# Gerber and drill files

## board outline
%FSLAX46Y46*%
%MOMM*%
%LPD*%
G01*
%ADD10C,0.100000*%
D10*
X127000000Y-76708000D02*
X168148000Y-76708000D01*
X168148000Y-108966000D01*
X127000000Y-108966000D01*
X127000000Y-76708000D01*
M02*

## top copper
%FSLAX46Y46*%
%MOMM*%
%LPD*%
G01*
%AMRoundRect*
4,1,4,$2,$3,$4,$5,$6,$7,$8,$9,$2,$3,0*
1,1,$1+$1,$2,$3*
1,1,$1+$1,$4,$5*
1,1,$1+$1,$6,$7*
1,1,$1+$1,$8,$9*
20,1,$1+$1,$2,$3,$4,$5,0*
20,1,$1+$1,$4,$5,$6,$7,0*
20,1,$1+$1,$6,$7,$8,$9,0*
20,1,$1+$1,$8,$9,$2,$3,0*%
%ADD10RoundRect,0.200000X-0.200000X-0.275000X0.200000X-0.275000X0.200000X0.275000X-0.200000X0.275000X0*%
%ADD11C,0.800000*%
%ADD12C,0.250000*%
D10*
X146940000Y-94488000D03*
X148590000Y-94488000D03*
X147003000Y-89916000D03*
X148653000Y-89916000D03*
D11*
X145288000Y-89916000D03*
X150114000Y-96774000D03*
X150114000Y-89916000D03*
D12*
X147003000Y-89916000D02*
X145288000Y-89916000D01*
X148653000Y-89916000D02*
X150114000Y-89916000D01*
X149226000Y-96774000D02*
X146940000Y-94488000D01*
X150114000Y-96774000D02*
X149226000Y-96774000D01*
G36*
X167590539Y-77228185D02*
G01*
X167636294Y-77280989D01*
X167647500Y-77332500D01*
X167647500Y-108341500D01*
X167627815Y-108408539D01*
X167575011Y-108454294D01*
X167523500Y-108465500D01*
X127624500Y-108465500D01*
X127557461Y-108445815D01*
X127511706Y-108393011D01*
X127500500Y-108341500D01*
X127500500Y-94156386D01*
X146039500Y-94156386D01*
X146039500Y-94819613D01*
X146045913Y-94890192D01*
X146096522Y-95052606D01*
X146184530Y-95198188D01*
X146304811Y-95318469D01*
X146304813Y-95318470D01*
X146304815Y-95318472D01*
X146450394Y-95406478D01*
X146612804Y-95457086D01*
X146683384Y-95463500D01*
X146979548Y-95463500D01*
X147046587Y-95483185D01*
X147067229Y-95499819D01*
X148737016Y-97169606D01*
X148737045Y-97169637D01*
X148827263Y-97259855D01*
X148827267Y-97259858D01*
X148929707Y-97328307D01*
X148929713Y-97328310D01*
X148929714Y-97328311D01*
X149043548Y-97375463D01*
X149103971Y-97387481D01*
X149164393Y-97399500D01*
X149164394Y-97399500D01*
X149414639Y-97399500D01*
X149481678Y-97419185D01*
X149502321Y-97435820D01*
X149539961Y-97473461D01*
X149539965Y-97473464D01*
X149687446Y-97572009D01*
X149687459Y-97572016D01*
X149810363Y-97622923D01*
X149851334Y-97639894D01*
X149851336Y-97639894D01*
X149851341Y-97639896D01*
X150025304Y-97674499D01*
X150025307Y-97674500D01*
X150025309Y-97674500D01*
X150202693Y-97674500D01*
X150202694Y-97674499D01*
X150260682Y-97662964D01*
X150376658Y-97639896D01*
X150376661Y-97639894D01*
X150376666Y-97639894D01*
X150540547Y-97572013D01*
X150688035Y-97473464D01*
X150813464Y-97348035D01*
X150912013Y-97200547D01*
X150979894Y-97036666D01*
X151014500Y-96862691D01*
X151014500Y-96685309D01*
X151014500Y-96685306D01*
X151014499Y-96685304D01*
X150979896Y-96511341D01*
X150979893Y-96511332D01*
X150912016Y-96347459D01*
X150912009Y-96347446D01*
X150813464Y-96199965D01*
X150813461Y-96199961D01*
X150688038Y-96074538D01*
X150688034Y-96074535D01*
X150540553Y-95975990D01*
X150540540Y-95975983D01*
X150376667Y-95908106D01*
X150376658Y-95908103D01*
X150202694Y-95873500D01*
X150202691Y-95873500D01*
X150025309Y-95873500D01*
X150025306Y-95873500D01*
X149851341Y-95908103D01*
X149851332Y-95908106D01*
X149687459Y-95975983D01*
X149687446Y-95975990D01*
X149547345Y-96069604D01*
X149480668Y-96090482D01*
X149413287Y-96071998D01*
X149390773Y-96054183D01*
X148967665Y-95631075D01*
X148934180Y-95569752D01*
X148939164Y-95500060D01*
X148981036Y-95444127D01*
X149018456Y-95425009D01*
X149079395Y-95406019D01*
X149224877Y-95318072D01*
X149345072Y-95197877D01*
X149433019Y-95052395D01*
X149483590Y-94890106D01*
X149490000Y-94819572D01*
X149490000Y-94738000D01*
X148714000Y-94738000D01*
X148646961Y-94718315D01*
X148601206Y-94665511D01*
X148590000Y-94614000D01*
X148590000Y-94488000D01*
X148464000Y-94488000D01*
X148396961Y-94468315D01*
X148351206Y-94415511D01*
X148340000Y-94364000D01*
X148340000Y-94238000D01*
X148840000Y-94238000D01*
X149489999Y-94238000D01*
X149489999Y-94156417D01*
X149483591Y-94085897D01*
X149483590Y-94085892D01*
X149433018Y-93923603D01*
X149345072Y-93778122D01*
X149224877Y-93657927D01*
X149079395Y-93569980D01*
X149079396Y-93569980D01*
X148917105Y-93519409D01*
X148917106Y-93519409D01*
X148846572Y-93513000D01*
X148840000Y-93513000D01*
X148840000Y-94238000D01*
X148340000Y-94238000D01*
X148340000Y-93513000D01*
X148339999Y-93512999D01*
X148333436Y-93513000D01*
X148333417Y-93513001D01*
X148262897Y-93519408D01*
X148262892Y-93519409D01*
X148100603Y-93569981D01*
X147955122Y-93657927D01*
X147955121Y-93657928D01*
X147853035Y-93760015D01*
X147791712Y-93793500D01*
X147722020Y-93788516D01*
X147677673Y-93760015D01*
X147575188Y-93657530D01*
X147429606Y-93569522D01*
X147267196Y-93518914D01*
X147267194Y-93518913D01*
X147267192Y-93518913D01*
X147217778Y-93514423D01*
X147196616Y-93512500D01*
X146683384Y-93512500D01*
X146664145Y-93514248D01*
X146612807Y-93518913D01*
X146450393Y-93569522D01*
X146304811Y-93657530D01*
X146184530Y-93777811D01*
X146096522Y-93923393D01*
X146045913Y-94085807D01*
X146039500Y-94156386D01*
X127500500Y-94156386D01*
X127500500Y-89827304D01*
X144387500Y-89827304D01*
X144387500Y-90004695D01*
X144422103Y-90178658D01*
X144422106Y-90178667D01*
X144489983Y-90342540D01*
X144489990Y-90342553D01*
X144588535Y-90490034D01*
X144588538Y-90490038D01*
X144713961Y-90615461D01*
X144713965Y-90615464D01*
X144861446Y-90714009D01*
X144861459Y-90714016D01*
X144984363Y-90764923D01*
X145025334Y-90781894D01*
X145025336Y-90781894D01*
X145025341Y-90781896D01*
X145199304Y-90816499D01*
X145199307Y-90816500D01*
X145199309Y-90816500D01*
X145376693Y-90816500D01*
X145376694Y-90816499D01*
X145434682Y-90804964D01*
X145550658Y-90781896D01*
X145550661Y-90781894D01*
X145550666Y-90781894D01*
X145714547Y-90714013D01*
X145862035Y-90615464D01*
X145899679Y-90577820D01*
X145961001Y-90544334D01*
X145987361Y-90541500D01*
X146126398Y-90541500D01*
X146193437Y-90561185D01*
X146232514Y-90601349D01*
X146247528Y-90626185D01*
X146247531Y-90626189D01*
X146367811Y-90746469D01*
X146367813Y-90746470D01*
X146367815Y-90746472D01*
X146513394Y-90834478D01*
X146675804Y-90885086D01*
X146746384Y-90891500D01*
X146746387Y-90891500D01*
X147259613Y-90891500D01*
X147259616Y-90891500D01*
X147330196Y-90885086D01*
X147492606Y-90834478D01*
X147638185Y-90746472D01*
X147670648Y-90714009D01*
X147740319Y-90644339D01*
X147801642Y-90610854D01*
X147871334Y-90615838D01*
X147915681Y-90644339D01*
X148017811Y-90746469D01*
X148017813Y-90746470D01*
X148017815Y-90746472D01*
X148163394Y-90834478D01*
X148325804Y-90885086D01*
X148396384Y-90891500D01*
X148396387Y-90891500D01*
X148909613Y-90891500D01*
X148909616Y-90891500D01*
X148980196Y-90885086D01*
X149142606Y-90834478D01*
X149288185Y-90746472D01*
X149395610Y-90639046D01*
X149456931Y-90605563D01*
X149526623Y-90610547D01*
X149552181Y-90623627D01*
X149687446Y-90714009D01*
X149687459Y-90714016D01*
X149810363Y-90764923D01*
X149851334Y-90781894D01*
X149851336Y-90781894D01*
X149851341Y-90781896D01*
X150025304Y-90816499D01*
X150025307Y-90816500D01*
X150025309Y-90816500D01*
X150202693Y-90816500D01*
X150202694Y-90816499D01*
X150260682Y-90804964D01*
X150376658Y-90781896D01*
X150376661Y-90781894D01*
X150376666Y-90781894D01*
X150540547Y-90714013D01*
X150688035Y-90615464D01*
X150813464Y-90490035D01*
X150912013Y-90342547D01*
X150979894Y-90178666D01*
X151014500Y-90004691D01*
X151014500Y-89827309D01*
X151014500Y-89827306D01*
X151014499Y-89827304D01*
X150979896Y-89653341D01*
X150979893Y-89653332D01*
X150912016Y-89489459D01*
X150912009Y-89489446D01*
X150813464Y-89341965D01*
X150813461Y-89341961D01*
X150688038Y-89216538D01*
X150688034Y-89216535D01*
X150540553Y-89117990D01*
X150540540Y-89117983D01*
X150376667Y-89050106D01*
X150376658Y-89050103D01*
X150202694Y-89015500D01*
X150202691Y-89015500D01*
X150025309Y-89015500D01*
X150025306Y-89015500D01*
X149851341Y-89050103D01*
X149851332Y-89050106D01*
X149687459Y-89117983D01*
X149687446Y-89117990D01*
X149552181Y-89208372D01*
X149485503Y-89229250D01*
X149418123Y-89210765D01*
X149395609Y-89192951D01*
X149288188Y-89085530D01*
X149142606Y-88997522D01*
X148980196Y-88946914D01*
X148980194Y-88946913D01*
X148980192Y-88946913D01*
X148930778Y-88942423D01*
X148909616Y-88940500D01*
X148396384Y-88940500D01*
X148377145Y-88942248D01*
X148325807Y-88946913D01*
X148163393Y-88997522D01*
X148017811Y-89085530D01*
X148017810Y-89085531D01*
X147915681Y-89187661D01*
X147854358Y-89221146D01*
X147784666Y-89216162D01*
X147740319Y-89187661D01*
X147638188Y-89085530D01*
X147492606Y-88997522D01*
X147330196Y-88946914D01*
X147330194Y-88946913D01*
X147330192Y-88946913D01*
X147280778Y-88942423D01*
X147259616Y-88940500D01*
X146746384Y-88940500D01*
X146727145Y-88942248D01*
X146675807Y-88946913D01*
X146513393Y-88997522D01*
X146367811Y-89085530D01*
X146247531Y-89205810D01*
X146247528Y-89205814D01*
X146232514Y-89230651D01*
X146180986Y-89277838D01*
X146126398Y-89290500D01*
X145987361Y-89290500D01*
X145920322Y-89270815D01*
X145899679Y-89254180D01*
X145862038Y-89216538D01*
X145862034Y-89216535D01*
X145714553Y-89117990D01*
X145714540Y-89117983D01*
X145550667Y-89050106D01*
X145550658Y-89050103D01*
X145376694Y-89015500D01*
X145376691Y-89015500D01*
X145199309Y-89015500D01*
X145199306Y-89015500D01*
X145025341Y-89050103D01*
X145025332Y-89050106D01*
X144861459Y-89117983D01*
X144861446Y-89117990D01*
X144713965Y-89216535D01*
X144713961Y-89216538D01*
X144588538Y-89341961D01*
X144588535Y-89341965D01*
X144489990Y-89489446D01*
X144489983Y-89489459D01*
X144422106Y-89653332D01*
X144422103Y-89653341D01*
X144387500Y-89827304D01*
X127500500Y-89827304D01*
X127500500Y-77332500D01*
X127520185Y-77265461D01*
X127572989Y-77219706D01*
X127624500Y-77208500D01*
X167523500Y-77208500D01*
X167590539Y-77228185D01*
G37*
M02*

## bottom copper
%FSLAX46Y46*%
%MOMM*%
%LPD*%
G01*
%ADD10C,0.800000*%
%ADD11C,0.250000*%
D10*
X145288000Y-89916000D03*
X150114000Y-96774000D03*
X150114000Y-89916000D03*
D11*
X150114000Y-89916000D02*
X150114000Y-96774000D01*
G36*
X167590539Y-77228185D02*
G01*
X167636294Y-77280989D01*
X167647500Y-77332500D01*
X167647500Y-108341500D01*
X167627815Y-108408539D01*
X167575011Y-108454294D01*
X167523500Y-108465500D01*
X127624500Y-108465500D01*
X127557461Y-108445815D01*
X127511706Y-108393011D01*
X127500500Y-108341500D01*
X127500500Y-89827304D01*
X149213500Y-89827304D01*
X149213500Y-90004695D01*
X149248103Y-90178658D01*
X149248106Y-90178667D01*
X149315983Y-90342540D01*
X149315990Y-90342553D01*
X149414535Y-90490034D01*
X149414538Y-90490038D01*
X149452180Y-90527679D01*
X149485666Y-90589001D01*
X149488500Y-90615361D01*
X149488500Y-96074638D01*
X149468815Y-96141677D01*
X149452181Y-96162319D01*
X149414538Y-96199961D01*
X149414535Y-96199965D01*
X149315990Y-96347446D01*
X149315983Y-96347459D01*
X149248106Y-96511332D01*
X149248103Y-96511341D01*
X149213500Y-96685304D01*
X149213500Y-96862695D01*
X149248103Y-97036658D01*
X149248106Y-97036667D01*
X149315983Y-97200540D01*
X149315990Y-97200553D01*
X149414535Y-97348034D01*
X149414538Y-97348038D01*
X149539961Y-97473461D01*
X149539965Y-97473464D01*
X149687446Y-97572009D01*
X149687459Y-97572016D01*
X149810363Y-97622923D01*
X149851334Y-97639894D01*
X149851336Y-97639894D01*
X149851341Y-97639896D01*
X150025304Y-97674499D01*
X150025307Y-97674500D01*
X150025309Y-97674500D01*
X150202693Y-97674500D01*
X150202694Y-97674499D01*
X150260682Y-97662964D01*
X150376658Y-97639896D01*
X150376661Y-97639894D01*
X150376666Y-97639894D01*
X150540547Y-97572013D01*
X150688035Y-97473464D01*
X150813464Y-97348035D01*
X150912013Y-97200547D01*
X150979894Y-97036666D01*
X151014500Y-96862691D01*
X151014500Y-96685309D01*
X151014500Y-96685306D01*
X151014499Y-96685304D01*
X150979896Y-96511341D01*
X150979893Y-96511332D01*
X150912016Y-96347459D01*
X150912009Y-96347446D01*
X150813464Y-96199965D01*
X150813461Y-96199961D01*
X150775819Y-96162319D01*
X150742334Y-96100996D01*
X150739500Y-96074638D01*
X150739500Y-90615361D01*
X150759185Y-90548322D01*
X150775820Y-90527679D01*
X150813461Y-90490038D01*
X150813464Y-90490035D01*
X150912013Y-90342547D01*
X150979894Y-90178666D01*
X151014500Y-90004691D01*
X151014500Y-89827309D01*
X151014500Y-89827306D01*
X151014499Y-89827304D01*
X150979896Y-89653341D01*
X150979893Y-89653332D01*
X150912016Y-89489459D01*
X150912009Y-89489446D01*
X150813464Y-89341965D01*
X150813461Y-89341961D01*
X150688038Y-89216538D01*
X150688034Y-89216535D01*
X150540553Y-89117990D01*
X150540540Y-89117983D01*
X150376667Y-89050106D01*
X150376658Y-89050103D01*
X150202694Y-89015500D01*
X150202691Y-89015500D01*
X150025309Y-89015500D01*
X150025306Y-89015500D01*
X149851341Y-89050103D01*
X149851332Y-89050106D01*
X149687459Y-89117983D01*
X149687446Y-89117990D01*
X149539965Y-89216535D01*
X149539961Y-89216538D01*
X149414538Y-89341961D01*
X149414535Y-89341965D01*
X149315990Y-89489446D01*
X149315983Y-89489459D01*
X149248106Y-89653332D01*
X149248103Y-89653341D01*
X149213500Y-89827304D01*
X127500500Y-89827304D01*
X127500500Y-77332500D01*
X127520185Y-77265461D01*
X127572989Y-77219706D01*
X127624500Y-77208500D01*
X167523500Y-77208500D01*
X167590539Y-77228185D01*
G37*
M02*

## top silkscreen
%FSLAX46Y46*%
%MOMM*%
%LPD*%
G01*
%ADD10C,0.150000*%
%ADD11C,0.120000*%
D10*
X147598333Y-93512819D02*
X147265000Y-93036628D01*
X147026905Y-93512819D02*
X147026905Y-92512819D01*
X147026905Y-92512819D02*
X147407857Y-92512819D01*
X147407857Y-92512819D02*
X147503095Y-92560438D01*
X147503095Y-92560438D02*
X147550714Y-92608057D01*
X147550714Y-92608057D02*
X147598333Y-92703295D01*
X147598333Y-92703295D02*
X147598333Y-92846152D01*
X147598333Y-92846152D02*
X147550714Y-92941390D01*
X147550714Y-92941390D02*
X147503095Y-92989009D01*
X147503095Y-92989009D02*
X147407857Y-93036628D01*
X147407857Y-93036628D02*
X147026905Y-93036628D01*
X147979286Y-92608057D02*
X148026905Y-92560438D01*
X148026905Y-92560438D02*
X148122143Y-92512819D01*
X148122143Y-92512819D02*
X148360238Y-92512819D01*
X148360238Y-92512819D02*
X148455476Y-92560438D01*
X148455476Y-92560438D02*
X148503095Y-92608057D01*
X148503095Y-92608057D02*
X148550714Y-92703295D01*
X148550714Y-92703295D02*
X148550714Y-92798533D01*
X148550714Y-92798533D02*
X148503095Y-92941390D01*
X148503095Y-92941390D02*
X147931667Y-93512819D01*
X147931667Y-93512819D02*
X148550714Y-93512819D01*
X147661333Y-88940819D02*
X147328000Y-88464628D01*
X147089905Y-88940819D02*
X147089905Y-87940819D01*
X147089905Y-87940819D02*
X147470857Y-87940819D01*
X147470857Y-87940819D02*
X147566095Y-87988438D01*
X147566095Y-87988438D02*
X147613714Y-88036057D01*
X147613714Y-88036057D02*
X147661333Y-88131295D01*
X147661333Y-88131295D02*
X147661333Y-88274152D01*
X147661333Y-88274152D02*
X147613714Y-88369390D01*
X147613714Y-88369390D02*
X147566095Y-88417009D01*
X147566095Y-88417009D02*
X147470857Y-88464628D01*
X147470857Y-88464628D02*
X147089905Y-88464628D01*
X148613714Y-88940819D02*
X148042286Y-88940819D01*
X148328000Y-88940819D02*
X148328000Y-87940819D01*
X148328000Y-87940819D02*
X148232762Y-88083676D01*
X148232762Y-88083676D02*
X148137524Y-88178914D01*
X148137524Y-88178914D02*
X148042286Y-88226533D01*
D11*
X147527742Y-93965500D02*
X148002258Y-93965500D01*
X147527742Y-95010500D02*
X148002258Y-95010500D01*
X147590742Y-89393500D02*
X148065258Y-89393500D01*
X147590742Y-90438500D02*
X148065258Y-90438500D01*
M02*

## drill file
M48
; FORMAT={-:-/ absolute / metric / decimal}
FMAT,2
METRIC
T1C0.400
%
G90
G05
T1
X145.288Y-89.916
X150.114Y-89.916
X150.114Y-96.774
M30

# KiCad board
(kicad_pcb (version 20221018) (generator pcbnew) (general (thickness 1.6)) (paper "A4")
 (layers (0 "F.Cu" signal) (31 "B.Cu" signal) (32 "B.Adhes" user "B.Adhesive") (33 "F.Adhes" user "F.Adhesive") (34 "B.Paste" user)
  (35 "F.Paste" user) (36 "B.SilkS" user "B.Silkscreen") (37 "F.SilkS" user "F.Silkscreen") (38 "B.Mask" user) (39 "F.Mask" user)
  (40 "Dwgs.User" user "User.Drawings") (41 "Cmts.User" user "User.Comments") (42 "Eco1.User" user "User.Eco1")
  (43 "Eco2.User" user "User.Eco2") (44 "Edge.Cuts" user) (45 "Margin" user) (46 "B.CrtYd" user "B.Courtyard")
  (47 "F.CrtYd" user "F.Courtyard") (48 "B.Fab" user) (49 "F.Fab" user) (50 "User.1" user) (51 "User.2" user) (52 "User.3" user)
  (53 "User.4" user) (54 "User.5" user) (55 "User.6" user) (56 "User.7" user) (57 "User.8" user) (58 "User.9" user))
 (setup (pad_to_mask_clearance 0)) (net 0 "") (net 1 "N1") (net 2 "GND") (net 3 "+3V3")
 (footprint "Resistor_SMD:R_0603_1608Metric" (layer "F.Cu") (at 147.765 94.488)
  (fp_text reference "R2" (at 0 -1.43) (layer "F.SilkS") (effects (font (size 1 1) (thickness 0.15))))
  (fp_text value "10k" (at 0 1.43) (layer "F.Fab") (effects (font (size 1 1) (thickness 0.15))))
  (fp_line (start -0.237258 -0.5225) (end 0.237258 -0.5225) (stroke (width 0.12) (type solid)) (layer "F.SilkS"))
  (fp_line (start -0.237258 0.5225) (end 0.237258 0.5225) (stroke (width 0.12) (type solid)) (layer "F.SilkS"))
  (pad "1" smd roundrect (at -0.825 0) (size 0.8 0.95) (layers "F.Cu" "F.Paste" "F.Mask") (roundrect_rratio 0.25) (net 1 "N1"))
  (pad "2" smd roundrect (at 0.825 0) (size 0.8 0.95) (layers "F.Cu" "F.Paste" "F.Mask") (roundrect_rratio 0.25) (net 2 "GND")))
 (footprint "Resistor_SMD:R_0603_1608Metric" (layer "F.Cu") (at 147.828 89.916)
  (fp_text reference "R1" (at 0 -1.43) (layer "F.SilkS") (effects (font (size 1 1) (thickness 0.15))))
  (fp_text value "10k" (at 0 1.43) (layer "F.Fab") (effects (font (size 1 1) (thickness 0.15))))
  (fp_line (start -0.237258 -0.5225) (end 0.237258 -0.5225) (stroke (width 0.12) (type solid)) (layer "F.SilkS"))
  (fp_line (start -0.237258 0.5225) (end 0.237258 0.5225) (stroke (width 0.12) (type solid)) (layer "F.SilkS"))
  (pad "1" smd roundrect (at -0.825 0) (size 0.8 0.95) (layers "F.Cu" "F.Paste" "F.Mask") (roundrect_rratio 0.25) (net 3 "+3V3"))
  (pad "2" smd roundrect (at 0.825 0) (size 0.8 0.95) (layers "F.Cu" "F.Paste" "F.Mask") (roundrect_rratio 0.25) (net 1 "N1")))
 (gr_rect (start 127 76.708) (end 168.148 108.966) (stroke (width 0.1) (type default)) (fill none) (layer "Edge.Cuts"))
 (segment (start 147.003 89.916) (end 145.288 89.916) (width 0.25) (layer "F.Cu") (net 3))
 (via (at 145.288 89.916) (size 0.8) (drill 0.4) (layers "F.Cu" "B.Cu") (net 3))
 (segment (start 148.653 89.916) (end 150.114 89.916) (width 0.25) (layer "F.Cu") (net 1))
 (segment (start 149.226 96.774) (end 146.94 94.488) (width 0.25) (layer "F.Cu") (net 1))
 (segment (start 150.114 96.774) (end 149.226 96.774) (width 0.25) (layer "F.Cu") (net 1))
 (via (at 150.114 96.774) (size 0.8) (drill 0.4) (layers "F.Cu" "B.Cu") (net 1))
 (via (at 150.114 89.916) (size 0.8) (drill 0.4) (layers "F.Cu" "B.Cu") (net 1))
 (segment (start 150.114 89.916) (end 150.114 96.774) (width 0.25) (layer "B.Cu") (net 1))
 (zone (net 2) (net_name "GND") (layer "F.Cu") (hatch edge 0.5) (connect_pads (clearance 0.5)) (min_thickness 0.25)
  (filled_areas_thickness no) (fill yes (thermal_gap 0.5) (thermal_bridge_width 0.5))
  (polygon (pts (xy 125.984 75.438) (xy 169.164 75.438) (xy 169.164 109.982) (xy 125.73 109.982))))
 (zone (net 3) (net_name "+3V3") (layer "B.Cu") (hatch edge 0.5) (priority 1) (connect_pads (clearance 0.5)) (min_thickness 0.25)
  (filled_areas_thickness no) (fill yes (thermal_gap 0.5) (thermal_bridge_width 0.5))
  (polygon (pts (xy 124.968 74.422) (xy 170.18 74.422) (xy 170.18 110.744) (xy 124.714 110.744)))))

